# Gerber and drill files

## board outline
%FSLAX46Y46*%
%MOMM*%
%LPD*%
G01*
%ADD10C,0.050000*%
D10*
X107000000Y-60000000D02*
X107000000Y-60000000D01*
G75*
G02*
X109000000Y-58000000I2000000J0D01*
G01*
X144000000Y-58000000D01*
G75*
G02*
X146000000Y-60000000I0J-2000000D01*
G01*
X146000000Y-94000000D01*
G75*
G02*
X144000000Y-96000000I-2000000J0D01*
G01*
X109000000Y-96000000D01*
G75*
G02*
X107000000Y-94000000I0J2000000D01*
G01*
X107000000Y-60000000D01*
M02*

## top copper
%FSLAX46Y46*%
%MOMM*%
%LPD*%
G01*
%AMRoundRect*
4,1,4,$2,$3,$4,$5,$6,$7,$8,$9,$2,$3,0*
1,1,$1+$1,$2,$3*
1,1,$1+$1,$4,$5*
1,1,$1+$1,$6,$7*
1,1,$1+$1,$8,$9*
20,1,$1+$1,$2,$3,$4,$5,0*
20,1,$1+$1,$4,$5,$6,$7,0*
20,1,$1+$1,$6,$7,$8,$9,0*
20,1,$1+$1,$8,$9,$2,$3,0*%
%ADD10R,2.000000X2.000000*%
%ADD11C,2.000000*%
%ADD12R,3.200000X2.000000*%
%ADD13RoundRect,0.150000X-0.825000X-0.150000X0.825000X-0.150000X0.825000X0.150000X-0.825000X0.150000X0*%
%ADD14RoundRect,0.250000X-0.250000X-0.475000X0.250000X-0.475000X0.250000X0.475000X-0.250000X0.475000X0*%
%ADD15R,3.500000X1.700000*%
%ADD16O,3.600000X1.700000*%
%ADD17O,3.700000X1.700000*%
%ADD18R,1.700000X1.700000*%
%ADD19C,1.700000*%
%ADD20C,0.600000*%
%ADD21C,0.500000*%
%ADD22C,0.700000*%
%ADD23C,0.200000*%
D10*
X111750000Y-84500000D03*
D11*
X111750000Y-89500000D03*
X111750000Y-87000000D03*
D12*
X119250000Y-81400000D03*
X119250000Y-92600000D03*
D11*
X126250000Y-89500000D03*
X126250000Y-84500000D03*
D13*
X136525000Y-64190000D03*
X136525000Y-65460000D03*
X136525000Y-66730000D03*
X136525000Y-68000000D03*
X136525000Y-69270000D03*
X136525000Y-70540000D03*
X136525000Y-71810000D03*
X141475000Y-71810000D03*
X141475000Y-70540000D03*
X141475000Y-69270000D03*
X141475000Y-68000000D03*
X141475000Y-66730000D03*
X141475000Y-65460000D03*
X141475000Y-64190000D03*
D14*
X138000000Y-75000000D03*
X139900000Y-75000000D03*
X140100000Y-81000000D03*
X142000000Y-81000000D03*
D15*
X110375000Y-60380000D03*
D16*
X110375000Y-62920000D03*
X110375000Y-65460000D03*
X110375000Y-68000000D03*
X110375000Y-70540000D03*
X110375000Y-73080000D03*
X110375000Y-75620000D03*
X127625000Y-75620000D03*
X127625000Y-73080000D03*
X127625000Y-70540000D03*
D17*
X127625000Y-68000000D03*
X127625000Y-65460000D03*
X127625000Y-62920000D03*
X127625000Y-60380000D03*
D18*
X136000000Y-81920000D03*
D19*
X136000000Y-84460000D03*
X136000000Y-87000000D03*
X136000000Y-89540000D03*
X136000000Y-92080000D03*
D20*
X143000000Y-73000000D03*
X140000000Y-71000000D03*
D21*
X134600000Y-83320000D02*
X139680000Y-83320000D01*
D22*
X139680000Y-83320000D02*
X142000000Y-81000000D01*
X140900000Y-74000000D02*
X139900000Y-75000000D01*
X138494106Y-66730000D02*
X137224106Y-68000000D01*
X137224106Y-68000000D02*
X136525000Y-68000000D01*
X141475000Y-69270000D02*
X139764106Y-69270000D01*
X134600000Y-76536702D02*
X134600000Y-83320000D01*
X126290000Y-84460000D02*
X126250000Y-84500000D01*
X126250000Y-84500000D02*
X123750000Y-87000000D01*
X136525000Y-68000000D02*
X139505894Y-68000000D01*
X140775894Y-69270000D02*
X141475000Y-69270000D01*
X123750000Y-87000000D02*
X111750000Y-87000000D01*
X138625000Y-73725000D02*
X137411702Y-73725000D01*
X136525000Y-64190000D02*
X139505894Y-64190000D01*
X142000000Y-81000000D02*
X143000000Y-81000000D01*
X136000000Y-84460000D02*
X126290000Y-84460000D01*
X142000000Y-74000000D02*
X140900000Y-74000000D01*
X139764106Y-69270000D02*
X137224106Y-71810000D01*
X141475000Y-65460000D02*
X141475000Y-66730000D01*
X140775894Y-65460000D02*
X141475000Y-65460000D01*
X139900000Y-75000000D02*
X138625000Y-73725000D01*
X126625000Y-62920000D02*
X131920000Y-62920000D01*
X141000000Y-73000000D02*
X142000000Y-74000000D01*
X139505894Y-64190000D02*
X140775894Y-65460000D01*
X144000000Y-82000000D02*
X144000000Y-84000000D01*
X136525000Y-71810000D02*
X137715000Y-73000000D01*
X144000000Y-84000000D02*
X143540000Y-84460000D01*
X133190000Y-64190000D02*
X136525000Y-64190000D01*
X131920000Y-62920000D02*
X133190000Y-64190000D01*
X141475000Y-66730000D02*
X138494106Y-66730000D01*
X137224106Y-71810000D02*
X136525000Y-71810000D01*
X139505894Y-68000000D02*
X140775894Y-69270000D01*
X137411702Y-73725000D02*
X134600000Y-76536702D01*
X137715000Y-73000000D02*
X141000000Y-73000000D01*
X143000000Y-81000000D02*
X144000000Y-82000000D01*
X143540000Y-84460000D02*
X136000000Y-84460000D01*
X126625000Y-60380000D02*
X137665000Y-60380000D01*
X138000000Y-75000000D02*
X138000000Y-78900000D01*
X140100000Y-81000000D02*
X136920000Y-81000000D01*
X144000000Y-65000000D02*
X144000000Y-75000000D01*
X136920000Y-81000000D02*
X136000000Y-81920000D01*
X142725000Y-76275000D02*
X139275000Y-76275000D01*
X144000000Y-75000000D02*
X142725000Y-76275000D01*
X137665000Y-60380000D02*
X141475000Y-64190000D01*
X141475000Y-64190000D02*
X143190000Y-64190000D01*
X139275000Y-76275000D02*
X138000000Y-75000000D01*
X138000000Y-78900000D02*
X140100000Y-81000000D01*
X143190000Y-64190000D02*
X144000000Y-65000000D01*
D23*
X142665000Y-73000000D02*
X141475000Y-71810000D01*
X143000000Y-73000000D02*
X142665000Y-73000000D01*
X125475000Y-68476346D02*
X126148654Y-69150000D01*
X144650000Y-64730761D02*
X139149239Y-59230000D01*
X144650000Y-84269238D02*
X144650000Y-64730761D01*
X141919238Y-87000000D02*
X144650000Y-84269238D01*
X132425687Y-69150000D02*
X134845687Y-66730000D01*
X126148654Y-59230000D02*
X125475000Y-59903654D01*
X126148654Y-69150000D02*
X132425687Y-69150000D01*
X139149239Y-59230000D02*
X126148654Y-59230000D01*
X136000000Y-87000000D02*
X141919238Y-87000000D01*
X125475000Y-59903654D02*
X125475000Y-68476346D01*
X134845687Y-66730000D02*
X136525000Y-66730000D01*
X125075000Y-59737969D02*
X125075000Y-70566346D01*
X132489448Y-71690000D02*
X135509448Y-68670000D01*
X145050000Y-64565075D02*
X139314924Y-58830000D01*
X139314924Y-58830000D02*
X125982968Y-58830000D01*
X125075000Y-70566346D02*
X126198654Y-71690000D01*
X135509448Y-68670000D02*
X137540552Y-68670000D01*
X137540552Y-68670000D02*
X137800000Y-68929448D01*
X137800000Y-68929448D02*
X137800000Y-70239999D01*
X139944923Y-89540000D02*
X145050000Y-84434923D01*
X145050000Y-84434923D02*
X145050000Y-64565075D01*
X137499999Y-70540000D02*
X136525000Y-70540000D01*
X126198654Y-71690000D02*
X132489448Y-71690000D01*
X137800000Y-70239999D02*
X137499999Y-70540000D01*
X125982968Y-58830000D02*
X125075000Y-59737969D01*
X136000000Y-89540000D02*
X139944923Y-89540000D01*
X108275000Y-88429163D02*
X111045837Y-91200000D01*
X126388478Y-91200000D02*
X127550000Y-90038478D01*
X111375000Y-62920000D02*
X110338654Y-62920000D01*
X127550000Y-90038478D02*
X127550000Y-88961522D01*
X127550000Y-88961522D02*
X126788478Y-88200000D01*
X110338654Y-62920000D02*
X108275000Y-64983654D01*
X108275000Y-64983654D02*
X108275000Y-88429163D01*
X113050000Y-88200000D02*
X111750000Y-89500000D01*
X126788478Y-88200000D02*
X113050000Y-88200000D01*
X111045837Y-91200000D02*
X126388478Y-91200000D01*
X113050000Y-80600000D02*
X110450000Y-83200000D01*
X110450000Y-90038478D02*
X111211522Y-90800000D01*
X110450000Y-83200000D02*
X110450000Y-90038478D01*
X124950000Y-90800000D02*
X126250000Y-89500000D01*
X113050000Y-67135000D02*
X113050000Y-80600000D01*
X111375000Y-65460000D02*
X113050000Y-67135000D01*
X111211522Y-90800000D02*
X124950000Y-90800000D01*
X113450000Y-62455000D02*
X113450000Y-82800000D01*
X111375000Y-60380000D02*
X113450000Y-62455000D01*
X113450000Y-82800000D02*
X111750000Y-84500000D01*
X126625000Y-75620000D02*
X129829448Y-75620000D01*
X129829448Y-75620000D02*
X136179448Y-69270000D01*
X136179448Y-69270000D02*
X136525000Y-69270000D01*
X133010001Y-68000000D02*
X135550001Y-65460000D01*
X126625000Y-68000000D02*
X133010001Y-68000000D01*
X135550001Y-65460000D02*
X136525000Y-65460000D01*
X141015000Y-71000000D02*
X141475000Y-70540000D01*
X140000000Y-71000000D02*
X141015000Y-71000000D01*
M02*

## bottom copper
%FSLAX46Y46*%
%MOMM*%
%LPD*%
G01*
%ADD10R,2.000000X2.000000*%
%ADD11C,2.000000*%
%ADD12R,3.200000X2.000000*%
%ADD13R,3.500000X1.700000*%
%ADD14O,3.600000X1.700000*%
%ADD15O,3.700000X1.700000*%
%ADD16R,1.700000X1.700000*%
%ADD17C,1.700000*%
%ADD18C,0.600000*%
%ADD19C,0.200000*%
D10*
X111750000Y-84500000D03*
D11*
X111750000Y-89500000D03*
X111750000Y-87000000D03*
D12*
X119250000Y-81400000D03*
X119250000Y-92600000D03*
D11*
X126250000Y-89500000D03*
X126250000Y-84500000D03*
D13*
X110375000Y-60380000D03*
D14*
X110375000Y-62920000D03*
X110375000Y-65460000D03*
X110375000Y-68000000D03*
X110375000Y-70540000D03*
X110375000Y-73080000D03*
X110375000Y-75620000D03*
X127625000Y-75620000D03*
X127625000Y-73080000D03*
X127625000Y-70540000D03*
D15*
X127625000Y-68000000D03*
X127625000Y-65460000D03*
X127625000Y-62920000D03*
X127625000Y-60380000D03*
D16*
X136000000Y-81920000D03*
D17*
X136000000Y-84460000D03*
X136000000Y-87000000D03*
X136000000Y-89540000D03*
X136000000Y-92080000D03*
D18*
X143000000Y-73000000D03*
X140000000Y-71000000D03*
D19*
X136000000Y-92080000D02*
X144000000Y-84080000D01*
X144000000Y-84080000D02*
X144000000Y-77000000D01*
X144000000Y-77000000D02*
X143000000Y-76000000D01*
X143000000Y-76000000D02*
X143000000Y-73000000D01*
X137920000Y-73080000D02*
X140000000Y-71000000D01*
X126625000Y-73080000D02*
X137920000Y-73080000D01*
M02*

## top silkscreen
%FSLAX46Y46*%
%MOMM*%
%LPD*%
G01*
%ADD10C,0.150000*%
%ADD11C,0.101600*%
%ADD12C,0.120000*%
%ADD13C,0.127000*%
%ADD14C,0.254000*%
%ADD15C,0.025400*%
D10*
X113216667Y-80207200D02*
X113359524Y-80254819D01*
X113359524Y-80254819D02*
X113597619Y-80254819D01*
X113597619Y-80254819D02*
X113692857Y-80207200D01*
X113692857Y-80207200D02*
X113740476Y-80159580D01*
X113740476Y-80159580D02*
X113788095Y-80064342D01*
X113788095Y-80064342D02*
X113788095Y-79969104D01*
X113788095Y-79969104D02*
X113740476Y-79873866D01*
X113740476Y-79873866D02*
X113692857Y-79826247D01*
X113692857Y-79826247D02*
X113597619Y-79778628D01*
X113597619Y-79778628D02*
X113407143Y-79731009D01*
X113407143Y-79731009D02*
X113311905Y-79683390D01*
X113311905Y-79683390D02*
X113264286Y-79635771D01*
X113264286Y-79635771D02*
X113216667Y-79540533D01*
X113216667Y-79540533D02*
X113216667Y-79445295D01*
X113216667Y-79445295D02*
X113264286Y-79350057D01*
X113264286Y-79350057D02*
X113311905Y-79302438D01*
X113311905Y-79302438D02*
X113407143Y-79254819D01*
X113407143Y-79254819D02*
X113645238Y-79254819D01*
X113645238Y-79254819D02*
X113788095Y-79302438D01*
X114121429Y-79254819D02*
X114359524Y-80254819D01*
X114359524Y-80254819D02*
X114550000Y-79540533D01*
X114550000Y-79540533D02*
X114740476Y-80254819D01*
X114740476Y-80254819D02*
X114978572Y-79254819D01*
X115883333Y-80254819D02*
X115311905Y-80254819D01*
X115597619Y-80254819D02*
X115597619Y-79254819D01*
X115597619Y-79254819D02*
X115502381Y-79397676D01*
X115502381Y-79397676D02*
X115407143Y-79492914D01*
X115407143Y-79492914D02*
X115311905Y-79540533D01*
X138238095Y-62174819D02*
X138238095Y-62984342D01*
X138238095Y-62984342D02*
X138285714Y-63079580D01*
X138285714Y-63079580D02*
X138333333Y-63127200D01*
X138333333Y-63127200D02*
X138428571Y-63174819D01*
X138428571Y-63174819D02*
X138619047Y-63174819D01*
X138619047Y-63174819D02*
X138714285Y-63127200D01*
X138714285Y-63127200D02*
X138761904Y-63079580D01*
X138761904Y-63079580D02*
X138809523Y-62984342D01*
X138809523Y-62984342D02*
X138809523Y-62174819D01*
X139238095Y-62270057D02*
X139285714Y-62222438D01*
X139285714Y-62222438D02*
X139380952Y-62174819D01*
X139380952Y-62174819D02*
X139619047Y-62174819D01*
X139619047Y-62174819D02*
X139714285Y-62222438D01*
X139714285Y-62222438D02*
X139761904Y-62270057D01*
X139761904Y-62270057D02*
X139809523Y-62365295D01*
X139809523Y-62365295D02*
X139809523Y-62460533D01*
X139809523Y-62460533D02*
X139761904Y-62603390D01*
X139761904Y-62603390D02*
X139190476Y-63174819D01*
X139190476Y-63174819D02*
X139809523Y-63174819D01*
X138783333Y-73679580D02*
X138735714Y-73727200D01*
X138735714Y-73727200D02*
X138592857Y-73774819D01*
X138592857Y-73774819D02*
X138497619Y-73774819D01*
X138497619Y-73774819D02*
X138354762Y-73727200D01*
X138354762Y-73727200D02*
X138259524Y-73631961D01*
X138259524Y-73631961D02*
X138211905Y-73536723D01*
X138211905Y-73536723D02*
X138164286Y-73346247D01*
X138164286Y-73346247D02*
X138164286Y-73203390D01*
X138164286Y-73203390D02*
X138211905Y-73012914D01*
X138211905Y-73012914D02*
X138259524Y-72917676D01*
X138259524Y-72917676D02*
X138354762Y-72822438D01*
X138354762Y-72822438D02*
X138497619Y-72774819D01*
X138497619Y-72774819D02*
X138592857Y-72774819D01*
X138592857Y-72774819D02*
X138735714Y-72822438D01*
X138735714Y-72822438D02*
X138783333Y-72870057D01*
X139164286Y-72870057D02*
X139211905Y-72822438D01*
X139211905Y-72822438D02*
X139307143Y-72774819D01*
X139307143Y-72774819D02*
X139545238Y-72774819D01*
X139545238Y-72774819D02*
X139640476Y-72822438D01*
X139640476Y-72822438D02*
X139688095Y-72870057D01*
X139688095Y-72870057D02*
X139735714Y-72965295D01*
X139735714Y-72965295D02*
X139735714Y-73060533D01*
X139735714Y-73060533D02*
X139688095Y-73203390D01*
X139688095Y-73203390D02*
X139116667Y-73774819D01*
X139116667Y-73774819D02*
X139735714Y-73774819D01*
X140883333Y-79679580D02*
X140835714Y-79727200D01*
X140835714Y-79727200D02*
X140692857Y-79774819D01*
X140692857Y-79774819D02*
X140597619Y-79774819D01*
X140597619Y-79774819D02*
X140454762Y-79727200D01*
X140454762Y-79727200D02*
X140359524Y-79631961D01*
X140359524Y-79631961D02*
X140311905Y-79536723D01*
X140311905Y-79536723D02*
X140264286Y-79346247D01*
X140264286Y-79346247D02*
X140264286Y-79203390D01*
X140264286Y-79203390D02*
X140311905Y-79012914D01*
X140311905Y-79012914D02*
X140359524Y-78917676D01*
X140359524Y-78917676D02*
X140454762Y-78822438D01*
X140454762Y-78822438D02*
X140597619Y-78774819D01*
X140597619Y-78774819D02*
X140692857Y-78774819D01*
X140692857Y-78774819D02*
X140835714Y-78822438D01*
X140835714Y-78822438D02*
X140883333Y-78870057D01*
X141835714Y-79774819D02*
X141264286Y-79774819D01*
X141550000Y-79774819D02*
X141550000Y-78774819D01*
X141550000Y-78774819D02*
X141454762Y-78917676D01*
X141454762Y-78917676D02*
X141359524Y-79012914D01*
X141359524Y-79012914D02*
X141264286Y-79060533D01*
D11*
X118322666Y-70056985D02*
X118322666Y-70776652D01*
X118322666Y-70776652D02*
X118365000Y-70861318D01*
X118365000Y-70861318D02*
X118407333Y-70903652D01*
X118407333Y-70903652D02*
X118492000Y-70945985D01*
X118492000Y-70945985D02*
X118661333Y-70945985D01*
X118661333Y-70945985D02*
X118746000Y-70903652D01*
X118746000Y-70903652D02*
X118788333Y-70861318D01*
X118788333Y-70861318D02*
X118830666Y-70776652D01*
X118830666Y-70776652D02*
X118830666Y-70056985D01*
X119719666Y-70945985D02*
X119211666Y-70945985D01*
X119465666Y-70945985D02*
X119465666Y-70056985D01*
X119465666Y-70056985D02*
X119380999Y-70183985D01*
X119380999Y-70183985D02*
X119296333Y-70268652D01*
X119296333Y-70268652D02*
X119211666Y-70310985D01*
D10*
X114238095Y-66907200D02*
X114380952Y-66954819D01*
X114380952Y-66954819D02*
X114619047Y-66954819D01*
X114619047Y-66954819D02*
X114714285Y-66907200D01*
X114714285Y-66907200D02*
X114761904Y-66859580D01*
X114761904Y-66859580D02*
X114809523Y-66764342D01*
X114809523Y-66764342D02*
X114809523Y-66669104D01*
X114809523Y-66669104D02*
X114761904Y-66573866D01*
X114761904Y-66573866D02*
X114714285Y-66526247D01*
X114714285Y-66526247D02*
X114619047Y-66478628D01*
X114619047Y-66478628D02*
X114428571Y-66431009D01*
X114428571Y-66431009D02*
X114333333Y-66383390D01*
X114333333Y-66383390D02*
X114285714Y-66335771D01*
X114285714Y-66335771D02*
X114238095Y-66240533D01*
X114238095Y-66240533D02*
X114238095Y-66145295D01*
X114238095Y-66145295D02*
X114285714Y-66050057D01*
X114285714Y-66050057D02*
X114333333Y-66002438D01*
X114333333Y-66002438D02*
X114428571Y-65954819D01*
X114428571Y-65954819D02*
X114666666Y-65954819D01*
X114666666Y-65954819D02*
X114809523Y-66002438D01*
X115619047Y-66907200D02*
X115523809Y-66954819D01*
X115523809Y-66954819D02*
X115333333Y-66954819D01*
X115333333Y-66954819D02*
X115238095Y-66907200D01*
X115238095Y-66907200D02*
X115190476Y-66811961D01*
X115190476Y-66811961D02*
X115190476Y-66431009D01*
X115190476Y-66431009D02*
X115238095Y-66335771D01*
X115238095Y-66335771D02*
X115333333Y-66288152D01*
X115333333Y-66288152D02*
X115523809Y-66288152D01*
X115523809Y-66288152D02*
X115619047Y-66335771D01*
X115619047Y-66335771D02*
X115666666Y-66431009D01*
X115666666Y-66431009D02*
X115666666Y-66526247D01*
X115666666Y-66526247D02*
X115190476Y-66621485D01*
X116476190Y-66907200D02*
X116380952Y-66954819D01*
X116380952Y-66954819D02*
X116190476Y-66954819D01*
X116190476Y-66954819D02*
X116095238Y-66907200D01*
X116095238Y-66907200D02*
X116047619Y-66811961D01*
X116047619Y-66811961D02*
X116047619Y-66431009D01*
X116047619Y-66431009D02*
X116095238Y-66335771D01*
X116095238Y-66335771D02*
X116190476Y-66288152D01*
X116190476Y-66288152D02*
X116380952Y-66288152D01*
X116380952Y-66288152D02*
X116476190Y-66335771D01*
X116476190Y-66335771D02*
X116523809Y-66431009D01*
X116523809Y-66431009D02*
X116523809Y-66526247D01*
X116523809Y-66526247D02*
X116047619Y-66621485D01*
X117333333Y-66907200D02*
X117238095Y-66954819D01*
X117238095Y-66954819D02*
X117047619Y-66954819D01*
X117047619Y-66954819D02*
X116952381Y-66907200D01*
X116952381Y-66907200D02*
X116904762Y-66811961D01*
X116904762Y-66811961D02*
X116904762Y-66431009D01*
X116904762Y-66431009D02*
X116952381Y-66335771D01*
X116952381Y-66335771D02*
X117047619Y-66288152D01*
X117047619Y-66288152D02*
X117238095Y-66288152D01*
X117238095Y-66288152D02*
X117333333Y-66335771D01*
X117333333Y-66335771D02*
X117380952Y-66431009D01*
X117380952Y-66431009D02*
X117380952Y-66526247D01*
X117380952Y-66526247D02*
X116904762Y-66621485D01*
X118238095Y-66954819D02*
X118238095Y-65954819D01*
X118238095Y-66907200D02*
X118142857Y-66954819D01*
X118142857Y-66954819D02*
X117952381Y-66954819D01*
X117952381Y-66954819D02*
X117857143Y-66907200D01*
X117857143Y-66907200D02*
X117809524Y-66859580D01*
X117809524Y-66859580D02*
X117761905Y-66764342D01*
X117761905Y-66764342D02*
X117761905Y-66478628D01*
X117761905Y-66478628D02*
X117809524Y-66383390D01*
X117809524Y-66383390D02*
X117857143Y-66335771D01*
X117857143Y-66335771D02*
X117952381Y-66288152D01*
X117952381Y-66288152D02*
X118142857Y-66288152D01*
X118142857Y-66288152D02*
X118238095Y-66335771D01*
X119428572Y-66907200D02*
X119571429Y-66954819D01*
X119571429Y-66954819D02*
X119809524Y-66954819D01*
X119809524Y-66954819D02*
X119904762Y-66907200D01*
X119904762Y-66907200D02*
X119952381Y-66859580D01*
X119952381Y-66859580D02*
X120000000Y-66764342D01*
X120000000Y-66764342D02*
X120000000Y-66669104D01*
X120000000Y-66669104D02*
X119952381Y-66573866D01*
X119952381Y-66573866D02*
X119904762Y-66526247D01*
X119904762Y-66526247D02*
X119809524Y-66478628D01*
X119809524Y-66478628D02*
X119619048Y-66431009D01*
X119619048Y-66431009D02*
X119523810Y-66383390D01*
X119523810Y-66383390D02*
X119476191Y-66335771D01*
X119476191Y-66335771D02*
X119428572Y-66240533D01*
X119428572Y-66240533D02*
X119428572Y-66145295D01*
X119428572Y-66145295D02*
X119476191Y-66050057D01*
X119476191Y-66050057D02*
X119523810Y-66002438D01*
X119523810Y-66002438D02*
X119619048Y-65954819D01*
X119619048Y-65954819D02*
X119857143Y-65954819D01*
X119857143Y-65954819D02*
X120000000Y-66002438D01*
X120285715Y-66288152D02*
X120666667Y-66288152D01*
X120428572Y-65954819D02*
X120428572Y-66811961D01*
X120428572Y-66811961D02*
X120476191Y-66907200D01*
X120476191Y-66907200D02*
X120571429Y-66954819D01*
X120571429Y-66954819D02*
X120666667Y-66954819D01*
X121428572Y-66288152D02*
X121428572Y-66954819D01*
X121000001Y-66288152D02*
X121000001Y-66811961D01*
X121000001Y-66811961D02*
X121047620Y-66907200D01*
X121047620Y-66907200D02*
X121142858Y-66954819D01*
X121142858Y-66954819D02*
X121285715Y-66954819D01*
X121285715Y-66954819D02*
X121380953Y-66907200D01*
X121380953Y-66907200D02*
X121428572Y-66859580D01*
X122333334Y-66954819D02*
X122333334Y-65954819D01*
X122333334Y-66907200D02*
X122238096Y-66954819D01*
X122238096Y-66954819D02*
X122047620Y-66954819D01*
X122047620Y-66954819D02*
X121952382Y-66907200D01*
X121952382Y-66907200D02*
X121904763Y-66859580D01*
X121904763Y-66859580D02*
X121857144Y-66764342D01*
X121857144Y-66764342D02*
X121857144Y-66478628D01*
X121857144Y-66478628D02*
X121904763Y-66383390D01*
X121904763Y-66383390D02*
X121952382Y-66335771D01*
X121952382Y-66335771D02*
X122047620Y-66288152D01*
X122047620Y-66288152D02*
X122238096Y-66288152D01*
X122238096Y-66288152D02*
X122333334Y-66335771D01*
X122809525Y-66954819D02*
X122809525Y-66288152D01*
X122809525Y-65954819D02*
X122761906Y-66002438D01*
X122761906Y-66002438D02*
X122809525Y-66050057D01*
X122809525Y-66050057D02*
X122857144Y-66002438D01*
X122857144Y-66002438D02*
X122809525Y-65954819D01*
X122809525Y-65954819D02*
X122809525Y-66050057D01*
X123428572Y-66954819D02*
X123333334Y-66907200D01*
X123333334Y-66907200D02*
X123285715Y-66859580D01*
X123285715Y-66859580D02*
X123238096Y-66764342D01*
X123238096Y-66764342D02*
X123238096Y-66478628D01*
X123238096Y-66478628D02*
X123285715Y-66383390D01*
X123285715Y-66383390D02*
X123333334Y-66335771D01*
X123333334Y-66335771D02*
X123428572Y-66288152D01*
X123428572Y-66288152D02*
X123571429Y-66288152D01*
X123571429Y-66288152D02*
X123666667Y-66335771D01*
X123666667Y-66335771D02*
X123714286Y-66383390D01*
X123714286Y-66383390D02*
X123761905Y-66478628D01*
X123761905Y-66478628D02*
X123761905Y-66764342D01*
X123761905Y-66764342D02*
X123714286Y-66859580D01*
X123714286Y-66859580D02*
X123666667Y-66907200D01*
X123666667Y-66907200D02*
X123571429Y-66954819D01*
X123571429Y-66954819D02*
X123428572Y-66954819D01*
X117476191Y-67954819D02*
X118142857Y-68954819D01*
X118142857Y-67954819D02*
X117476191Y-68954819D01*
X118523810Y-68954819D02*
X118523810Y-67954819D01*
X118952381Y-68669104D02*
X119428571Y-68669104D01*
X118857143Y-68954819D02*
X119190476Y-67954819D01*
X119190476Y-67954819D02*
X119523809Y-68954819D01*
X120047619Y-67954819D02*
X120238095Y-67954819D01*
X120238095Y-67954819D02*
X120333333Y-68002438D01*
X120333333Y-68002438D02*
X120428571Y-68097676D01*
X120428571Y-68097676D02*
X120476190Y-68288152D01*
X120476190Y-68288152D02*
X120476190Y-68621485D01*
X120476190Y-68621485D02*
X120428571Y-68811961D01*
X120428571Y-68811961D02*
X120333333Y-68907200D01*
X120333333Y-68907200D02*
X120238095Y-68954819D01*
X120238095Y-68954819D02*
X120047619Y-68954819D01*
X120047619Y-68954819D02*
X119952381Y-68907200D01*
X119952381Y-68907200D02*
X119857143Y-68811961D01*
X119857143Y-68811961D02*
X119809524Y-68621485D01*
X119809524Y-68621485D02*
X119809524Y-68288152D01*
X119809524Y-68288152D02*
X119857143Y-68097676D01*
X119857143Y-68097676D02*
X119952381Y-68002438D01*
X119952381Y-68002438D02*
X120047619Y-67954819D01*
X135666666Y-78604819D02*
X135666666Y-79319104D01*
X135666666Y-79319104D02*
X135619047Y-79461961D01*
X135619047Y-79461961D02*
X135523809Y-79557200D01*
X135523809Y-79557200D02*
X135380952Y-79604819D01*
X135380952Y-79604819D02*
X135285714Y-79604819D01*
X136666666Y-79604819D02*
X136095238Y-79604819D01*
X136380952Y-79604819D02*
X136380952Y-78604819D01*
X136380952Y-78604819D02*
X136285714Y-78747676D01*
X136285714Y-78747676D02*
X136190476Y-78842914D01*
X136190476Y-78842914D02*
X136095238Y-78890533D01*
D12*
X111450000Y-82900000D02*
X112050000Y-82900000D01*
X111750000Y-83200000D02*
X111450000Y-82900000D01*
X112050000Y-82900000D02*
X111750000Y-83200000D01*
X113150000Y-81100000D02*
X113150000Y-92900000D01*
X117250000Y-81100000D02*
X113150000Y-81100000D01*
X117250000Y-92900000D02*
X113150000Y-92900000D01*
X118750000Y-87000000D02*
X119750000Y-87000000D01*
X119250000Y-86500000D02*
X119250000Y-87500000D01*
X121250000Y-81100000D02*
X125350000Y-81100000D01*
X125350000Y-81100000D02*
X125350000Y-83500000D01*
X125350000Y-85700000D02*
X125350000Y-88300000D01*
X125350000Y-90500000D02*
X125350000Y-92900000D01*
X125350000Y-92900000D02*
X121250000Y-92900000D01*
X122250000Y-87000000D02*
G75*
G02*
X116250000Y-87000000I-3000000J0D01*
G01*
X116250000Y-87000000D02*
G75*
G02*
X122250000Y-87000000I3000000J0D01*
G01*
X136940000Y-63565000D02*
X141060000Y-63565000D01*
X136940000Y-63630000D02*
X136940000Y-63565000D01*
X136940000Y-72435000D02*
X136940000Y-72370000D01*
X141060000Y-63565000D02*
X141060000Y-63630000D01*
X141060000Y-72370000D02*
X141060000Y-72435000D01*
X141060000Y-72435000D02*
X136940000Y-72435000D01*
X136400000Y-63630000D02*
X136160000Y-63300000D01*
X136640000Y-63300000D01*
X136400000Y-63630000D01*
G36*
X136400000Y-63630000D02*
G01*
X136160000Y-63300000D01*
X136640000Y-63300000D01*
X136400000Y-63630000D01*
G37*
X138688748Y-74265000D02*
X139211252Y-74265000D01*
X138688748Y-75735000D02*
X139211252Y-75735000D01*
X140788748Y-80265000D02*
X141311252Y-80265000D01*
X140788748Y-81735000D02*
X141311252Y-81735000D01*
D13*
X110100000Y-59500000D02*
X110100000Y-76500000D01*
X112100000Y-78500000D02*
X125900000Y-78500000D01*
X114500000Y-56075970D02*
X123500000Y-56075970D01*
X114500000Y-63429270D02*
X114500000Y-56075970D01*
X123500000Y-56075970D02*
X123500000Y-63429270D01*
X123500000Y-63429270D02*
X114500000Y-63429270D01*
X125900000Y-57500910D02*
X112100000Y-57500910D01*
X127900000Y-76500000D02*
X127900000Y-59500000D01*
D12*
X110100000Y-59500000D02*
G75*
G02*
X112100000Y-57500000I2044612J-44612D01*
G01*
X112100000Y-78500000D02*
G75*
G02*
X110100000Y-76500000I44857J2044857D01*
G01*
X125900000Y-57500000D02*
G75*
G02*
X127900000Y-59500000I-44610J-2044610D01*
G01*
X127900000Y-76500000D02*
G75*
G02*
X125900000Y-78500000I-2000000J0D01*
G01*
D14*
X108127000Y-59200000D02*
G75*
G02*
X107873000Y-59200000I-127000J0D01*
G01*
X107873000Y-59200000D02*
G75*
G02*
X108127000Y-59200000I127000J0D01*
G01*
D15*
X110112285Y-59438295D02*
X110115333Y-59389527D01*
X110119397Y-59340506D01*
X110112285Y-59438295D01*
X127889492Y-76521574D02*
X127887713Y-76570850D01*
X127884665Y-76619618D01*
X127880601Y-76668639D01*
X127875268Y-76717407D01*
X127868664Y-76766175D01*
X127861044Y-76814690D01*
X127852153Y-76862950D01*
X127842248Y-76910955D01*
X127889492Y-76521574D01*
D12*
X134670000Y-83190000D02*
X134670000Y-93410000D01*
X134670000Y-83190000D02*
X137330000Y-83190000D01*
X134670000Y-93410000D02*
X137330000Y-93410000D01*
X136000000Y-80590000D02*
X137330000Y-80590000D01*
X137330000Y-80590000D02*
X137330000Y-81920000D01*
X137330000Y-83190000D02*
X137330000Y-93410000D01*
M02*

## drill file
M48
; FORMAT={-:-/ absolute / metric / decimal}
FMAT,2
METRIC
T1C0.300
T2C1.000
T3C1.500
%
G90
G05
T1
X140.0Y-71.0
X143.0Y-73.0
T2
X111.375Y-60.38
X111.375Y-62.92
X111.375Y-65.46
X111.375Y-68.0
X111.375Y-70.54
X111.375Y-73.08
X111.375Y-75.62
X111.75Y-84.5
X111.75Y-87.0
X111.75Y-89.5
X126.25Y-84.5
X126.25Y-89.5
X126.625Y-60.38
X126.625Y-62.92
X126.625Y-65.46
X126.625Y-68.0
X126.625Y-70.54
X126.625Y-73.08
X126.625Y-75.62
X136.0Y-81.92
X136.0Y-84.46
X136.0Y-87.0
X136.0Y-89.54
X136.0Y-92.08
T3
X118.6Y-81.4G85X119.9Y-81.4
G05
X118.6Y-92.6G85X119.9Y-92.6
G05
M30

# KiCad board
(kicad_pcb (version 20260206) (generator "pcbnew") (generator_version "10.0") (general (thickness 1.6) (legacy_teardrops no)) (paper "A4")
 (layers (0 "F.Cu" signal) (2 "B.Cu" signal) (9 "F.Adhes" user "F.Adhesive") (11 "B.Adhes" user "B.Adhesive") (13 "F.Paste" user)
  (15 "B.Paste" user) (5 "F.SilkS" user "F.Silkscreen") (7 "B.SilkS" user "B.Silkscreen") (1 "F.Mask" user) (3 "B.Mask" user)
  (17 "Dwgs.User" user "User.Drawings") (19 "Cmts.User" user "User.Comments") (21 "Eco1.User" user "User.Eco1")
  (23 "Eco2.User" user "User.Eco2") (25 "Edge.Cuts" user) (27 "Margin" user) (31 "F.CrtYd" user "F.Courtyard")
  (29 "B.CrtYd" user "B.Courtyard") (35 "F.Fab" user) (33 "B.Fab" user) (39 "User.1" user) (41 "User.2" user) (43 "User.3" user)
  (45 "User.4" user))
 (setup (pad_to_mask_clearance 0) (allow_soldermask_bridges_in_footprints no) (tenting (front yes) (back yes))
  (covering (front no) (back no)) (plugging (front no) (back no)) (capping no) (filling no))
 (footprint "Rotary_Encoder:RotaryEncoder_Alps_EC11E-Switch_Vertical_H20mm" (layer "F.Cu") (at 111.75 84.5)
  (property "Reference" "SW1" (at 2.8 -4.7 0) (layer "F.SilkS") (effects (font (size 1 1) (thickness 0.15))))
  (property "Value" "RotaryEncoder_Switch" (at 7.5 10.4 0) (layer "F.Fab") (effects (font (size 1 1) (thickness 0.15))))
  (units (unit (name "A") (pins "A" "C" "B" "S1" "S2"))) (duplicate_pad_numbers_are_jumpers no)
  (fp_line (start -0.3 -1.6) (end 0.3 -1.6) (stroke (width 0.12) (type solid)) (layer "F.SilkS"))
  (fp_line (start 0 -1.3) (end -0.3 -1.6) (stroke (width 0.12) (type solid)) (layer "F.SilkS"))
  (fp_line (start 0.3 -1.6) (end 0 -1.3) (stroke (width 0.12) (type solid)) (layer "F.SilkS"))
  (fp_line (start 1.4 -3.4) (end 1.4 8.4) (stroke (width 0.12) (type solid)) (layer "F.SilkS"))
  (fp_line (start 5.5 -3.4) (end 1.4 -3.4) (stroke (width 0.12) (type solid)) (layer "F.SilkS"))
  (fp_line (start 5.5 8.4) (end 1.4 8.4) (stroke (width 0.12) (type solid)) (layer "F.SilkS"))
  (fp_line (start 7 2.5) (end 8 2.5) (stroke (width 0.12) (type solid)) (layer "F.SilkS"))
  (fp_line (start 7.5 2) (end 7.5 3) (stroke (width 0.12) (type solid)) (layer "F.SilkS"))
  (fp_line (start 9.5 -3.4) (end 13.6 -3.4) (stroke (width 0.12) (type solid)) (layer "F.SilkS"))
  (fp_line (start 13.6 -3.4) (end 13.6 -1) (stroke (width 0.12) (type solid)) (layer "F.SilkS"))
  (fp_line (start 13.6 1.2) (end 13.6 3.8) (stroke (width 0.12) (type solid)) (layer "F.SilkS"))
  (fp_line (start 13.6 6) (end 13.6 8.4) (stroke (width 0.12) (type solid)) (layer "F.SilkS"))
  (fp_line (start 13.6 8.4) (end 9.5 8.4) (stroke (width 0.12) (type solid)) (layer "F.SilkS"))
  (fp_circle (center 7.5 2.5) (end 10.5 2.5) (stroke (width 0.12) (type solid)) (fill no) (layer "F.SilkS"))
  (pad "A" thru_hole rect (at 0 0) (size 2 2) (drill 1) (layers "*.Cu" "*.Mask") (remove_unused_layers no) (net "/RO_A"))
  (pad "B" thru_hole circle (at 0 5) (size 2 2) (drill 1) (layers "*.Cu" "*.Mask") (remove_unused_layers no) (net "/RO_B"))
  (pad "C" thru_hole circle (at 0 2.5) (size 2 2) (drill 1) (layers "*.Cu" "*.Mask") (remove_unused_layers no) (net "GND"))
  (pad "MP" thru_hole rect (at 7.5 -3.1) (size 3.2 2) (drill oval 2.8 1.5) (layers "*.Cu" "*.Mask") (remove_unused_layers no))
  (pad "MP" thru_hole rect (at 7.5 8.1) (size 3.2 2) (drill oval 2.8 1.5) (layers "*.Cu" "*.Mask") (remove_unused_layers no))
  (pad "S1" thru_hole circle (at 14.5 5) (size 2 2) (drill 1) (layers "*.Cu" "*.Mask") (remove_unused_layers no) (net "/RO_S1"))
  (pad "S2" thru_hole circle (at 14.5 0) (size 2 2) (drill 1) (layers "*.Cu" "*.Mask") (remove_unused_layers no) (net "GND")))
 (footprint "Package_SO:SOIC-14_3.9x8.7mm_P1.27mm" (layer "F.Cu") (at 139 68)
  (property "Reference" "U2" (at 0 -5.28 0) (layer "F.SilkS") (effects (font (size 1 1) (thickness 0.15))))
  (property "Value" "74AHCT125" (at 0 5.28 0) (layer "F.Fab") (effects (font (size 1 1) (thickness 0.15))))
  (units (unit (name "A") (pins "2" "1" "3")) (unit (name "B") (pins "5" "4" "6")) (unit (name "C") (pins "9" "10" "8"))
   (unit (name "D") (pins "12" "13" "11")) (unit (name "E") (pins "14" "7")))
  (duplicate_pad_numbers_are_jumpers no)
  (fp_line (start -2.06 -4.435) (end 2.06 -4.435) (stroke (width 0.12) (type solid)) (layer "F.SilkS"))
  (fp_line (start -2.06 -4.37) (end -2.06 -4.435) (stroke (width 0.12) (type solid)) (layer "F.SilkS"))
  (fp_line (start -2.06 4.435) (end -2.06 4.37) (stroke (width 0.12) (type solid)) (layer "F.SilkS"))
  (fp_line (start 2.06 -4.435) (end 2.06 -4.37) (stroke (width 0.12) (type solid)) (layer "F.SilkS"))
  (fp_line (start 2.06 4.37) (end 2.06 4.435) (stroke (width 0.12) (type solid)) (layer "F.SilkS"))
  (fp_line (start 2.06 4.435) (end -2.06 4.435) (stroke (width 0.12) (type solid)) (layer "F.SilkS"))
  (fp_poly (pts (xy -2.6 -4.37) (xy -2.84 -4.7) (xy -2.36 -4.7)) (stroke (width 0.12) (type solid)) (fill yes) (layer "F.SilkS"))
  (pad "1" smd roundrect (at -2.475 -3.81) (size 1.95 0.6) (layers "F.Cu" "F.Mask" "F.Paste") (roundrect_rratio 0.25) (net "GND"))
  (pad "2" smd roundrect (at -2.475 -2.54) (size 1.95 0.6) (layers "F.Cu" "F.Mask" "F.Paste") (roundrect_rratio 0.25) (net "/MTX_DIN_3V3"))
  (pad "3" smd roundrect (at -2.475 -1.27) (size 1.95 0.6) (layers "F.Cu" "F.Mask" "F.Paste") (roundrect_rratio 0.25) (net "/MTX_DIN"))
  (pad "4" smd roundrect (at -2.475 0) (size 1.95 0.6) (layers "F.Cu" "F.Mask" "F.Paste") (roundrect_rratio 0.25) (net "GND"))
  (pad "5" smd roundrect (at -2.475 1.27) (size 1.95 0.6) (layers "F.Cu" "F.Mask" "F.Paste") (roundrect_rratio 0.25) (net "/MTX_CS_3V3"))
  (pad "6" smd roundrect (at -2.475 2.54) (size 1.95 0.6) (layers "F.Cu" "F.Mask" "F.Paste") (roundrect_rratio 0.25) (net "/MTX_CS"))
  (pad "7" smd roundrect (at -2.475 3.81) (size 1.95 0.6) (layers "F.Cu" "F.Mask" "F.Paste") (roundrect_rratio 0.25) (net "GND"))
  (pad "8" smd roundrect (at 2.475 3.81) (size 1.95 0.6) (layers "F.Cu" "F.Mask" "F.Paste") (roundrect_rratio 0.25) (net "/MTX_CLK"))
  (pad "9" smd roundrect (at 2.475 2.54) (size 1.95 0.6) (layers "F.Cu" "F.Mask" "F.Paste") (roundrect_rratio 0.25) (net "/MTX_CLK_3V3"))
  (pad "10" smd roundrect (at 2.475 1.27) (size 1.95 0.6) (layers "F.Cu" "F.Mask" "F.Paste") (roundrect_rratio 0.25) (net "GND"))
  (pad "11" smd roundrect (at 2.475 0) (size 1.95 0.6) (layers "F.Cu" "F.Mask" "F.Paste") (roundrect_rratio 0.25)
   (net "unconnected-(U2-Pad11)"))
  (pad "12" smd roundrect (at 2.475 -1.27) (size 1.95 0.6) (layers "F.Cu" "F.Mask" "F.Paste") (roundrect_rratio 0.25) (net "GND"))
  (pad "13" smd roundrect (at 2.475 -2.54) (size 1.95 0.6) (layers "F.Cu" "F.Mask" "F.Paste") (roundrect_rratio 0.25) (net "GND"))
  (pad "14" smd roundrect (at 2.475 -3.81) (size 1.95 0.6) (layers "F.Cu" "F.Mask" "F.Paste") (roundrect_rratio 0.25) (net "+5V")))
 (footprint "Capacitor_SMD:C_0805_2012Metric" (layer "F.Cu") (at 138.95 75)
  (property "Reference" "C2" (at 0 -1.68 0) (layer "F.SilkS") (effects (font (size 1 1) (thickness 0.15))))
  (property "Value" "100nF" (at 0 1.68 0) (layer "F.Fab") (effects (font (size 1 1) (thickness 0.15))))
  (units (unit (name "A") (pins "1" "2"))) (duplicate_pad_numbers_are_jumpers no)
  (fp_line (start -0.261252 -0.735) (end 0.261252 -0.735) (stroke (width 0.12) (type solid)) (layer "F.SilkS"))
  (fp_line (start -0.261252 0.735) (end 0.261252 0.735) (stroke (width 0.12) (type solid)) (layer "F.SilkS"))
  (pad "1" smd roundrect (at -0.95 0) (size 1 1.45) (layers "F.Cu" "F.Mask" "F.Paste") (roundrect_rratio 0.25) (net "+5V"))
  (pad "2" smd roundrect (at 0.95 0) (size 1 1.45) (layers "F.Cu" "F.Mask" "F.Paste") (roundrect_rratio 0.25) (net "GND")))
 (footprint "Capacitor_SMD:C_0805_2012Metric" (layer "F.Cu") (at 141.05 81)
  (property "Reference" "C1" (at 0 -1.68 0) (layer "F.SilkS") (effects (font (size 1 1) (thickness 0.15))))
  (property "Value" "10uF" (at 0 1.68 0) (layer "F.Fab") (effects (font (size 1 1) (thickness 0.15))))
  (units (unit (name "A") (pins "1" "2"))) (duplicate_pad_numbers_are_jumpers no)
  (fp_line (start -0.261252 -0.735) (end 0.261252 -0.735) (stroke (width 0.12) (type solid)) (layer "F.SilkS"))
  (fp_line (start -0.261252 0.735) (end 0.261252 0.735) (stroke (width 0.12) (type solid)) (layer "F.SilkS"))
  (pad "1" smd roundrect (at -0.95 0) (size 1 1.45) (layers "F.Cu" "F.Mask" "F.Paste") (roundrect_rratio 0.25) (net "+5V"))
  (pad "2" smd roundrect (at 0.95 0) (size 1 1.45) (layers "F.Cu" "F.Mask" "F.Paste") (roundrect_rratio 0.25) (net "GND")))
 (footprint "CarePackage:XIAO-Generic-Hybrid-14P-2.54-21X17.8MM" (layer "F.Cu") (at 119 68)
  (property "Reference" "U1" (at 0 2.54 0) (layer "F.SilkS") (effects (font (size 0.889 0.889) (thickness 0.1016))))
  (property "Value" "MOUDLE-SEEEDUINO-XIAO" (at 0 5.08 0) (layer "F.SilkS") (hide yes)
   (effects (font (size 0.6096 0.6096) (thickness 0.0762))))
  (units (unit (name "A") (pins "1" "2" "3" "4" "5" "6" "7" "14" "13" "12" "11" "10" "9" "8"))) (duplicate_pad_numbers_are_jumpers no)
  (fp_line (start -8.9 -8.5) (end -8.9 8.5) (stroke (width 0.127) (type solid)) (layer "F.SilkS"))
  (fp_line (start -6.9 10.5) (end 6.9 10.5) (stroke (width 0.127) (type solid)) (layer "F.SilkS"))
  (fp_line (start -4.5 -11.92403) (end 4.5 -11.92403) (stroke (width 0.127) (type solid)) (layer "F.SilkS"))
  (fp_line (start -4.5 -4.57073) (end -4.5 -11.92403) (stroke (width 0.127) (type solid)) (layer "F.SilkS"))
  (fp_line (start 4.5 -11.92403) (end 4.5 -4.57073) (stroke (width 0.127) (type solid)) (layer "F.SilkS"))
  (fp_line (start 4.5 -4.57073) (end -4.5 -4.57073) (stroke (width 0.127) (type solid)) (layer "F.SilkS"))
  (fp_line (start 6.9 -10.49909) (end -6.9 -10.49909) (stroke (width 0.127) (type solid)) (layer "F.SilkS"))
  (fp_line (start 8.9 8.5) (end 8.9 -8.5) (stroke (width 0.127) (type solid)) (layer "F.SilkS"))
  (fp_arc (start -8.9 -8.5) (mid -8.301491 -9.901491) (end -6.9 -10.5) (stroke (width 0.12) (type solid)) (layer "F.SilkS"))
  (fp_arc (start -6.9 10.5) (mid -8.301423 9.901423) (end -8.9 8.5) (stroke (width 0.12) (type solid)) (layer "F.SilkS"))
  (fp_arc (start 6.9 -10.5) (mid 8.301491 -9.901491) (end 8.9 -8.5) (stroke (width 0.12) (type solid)) (layer "F.SilkS"))
  (fp_arc (start 8.9 8.5) (mid 8.314214 9.914214) (end 6.9 10.5) (stroke (width 0.12) (type solid)) (layer "F.SilkS"))
  (fp_circle (center -11 -8.8) (end -11 -9.054) (stroke (width 0) (type solid)) (fill yes) (layer "F.SilkS"))
  (fp_poly
   (pts (xy -8.887715 -8.561705) (xy -8.884667 -8.610473) (xy -8.880603 -8.659494)) (stroke (width 0.0254) (type solid)) (fill no)
   (layer "F.SilkS"))
  (fp_poly
   (pts (xy 8.889492 8.521574) (xy 8.887713 8.57085) (xy 8.884665 8.619618) (xy 8.880601 8.668639) (xy 8.875268 8.717407)
    (xy 8.868664 8.766175) (xy 8.861044 8.81469) (xy 8.852153 8.86295) (xy 8.842248 8.910955))
   (stroke (width 0.0254) (type solid)) (fill no) (layer "F.SilkS"))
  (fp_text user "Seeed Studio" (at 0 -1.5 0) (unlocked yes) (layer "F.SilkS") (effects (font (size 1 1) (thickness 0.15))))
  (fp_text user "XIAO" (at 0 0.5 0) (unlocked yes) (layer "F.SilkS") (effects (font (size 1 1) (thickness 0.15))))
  (pad "1" thru_hole rect (at -7.625 -7.62) (size 3.5 1.7) (drill 1 (offset -1 0)) (layers "*.Cu" "*.Mask") (remove_unused_layers no)
   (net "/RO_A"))
  (pad "2" thru_hole oval (at -7.625 -5.08) (size 3.6 1.7) (drill 1 (offset -1 0)) (layers "*.Cu" "*.Mask") (remove_unused_layers no)
   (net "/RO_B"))
  (pad "3" thru_hole oval (at -7.625 -2.54) (size 3.6 1.7) (drill 1 (offset -1 0)) (layers "*.Cu" "*.Mask") (remove_unused_layers no)
   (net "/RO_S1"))
  (pad "4" thru_hole oval (at -7.625 0) (size 3.6 1.7) (drill 1 (offset -1 0)) (layers "*.Cu" "*.Mask") (remove_unused_layers no)
   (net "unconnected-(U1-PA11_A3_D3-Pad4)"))
  (pad "5" thru_hole oval (at -7.625 2.54) (size 3.6 1.7) (drill 1 (offset -1 0)) (layers "*.Cu" "*.Mask") (remove_unused_layers no)
   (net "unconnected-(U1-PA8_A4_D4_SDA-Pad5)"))
  (pad "6" thru_hole oval (at -7.625 5.08 180) (size 3.6 1.7) (drill 1 (offset 1 0)) (layers "*.Cu" "*.Mask") (remove_unused_layers no)
   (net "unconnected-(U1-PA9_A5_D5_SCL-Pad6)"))
  (pad "7" thru_hole oval (at -7.625 7.62) (size 3.6 1.7) (drill 1 (offset -1 0)) (layers "*.Cu" "*.Mask") (remove_unused_layers no)
   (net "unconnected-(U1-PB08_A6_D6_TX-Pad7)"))
  (pad "8" thru_hole oval (at 7.625 7.62) (size 3.6 1.7) (drill 1 (offset 1 0)) (layers "*.Cu" "*.Mask") (remove_unused_layers no)
   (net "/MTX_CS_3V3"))
  (pad "9" thru_hole oval (at 7.625 5.08) (size 3.6 1.7) (drill 1 (offset 1 0)) (layers "*.Cu" "*.Mask") (remove_unused_layers no)
   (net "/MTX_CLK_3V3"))
  (pad "10" thru_hole oval (at 7.625 2.54) (size 3.6 1.7) (drill 1 (offset 1 0)) (layers "*.Cu" "*.Mask") (remove_unused_layers no)
   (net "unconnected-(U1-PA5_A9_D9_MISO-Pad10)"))
  (pad "11" thru_hole oval (at 7.625 0) (size 3.7 1.7) (drill 1 (offset 1 0)) (layers "*.Cu" "*.Mask") (remove_unused_layers no)
   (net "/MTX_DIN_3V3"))
  (pad "12" thru_hole oval (at 7.625 -2.54) (size 3.7 1.7) (drill 1 (offset 1 0)) (layers "*.Cu" "*.Mask") (remove_unused_layers no)
   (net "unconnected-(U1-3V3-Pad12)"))
  (pad "13" thru_hole oval (at 7.625 -5.08) (size 3.7 1.7) (drill 1 (offset 1 0)) (layers "*.Cu" "*.Mask") (remove_unused_layers no)
   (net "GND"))
  (pad "14" thru_hole oval (at 7.625 -7.62) (size 3.7 1.7) (drill 1 (offset 1 0)) (layers "*.Cu" "*.Mask") (remove_unused_layers no)
   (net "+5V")))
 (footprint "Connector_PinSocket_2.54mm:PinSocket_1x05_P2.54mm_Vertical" (layer "F.Cu") (at 136 81.92)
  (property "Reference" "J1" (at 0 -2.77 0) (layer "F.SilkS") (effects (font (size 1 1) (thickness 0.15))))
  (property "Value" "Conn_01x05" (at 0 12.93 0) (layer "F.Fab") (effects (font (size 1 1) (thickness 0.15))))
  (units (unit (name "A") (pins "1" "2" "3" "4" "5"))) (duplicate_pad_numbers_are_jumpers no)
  (fp_line (start -1.33 1.27) (end -1.33 11.49) (stroke (width 0.12) (type solid)) (layer "F.SilkS"))
  (fp_line (start -1.33 1.27) (end 1.33 1.27) (stroke (width 0.12) (type solid)) (layer "F.SilkS"))
  (fp_line (start -1.33 11.49) (end 1.33 11.49) (stroke (width 0.12) (type solid)) (layer "F.SilkS"))
  (fp_line (start 0 -1.33) (end 1.33 -1.33) (stroke (width 0.12) (type solid)) (layer "F.SilkS"))
  (fp_line (start 1.33 -1.33) (end 1.33 0) (stroke (width 0.12) (type solid)) (layer "F.SilkS"))
  (fp_line (start 1.33 1.27) (end 1.33 11.49) (stroke (width 0.12) (type solid)) (layer "F.SilkS"))
  (pad "1" thru_hole rect (at 0 0) (size 1.7 1.7) (drill 1) (layers "*.Cu" "*.Mask") (remove_unused_layers no) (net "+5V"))
  (pad "2" thru_hole circle (at 0 2.54) (size 1.7 1.7) (drill 1) (layers "*.Cu" "*.Mask") (remove_unused_layers no) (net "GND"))
  (pad "3" thru_hole circle (at 0 5.08) (size 1.7 1.7) (drill 1) (layers "*.Cu" "*.Mask") (remove_unused_layers no) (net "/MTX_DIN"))
  (pad "4" thru_hole circle (at 0 7.62) (size 1.7 1.7) (drill 1) (layers "*.Cu" "*.Mask") (remove_unused_layers no) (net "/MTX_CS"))
  (pad "5" thru_hole circle (at 0 10.16) (size 1.7 1.7) (drill 1) (layers "*.Cu" "*.Mask") (remove_unused_layers no) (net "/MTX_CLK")))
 (gr_rect (start 107 58) (end 146 96) (radius 2) (stroke (width 0.05) (type default)) (fill no) (layer "Edge.Cuts"))
 (segment (start 134.6 83.32) (end 139.68 83.32) (width 0.5) (layer "F.Cu") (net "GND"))
 (segment (start 139.68 83.32) (end 142 81) (width 0.7) (layer "F.Cu") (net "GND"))
 (segment (start 140.9 74) (end 139.9 75) (width 0.7) (layer "F.Cu") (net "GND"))
 (segment (start 138.494106 66.73) (end 137.224106 68) (width 0.7) (layer "F.Cu") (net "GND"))
 (segment (start 137.224106 68) (end 136.525 68) (width 0.7) (layer "F.Cu") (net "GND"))
 (segment (start 141.475 69.27) (end 139.764106 69.27) (width 0.7) (layer "F.Cu") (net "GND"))
 (segment (start 134.6 76.536702) (end 134.6 83.32) (width 0.7) (layer "F.Cu") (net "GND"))
 (segment (start 126.29 84.46) (end 126.25 84.5) (width 0.7) (layer "F.Cu") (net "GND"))
 (segment (start 126.25 84.5) (end 123.75 87) (width 0.7) (layer "F.Cu") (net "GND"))
 (segment (start 136.525 68) (end 139.505894 68) (width 0.7) (layer "F.Cu") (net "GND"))
 (segment (start 140.775894 69.27) (end 141.475 69.27) (width 0.7) (layer "F.Cu") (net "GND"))
 (segment (start 123.75 87) (end 111.75 87) (width 0.7) (layer "F.Cu") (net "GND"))
 (segment (start 138.625 73.725) (end 137.411702 73.725) (width 0.7) (layer "F.Cu") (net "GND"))
 (segment (start 136.525 64.19) (end 139.505894 64.19) (width 0.7) (layer "F.Cu") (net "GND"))
 (segment (start 142 81) (end 143 81) (width 0.7) (layer "F.Cu") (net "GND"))
 (segment (start 136 84.46) (end 126.29 84.46) (width 0.7) (layer "F.Cu") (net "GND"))
 (segment (start 142 74) (end 140.9 74) (width 0.7) (layer "F.Cu") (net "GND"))
 (segment (start 139.764106 69.27) (end 137.224106 71.81) (width 0.7) (layer "F.Cu") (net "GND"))
 (segment (start 141.475 65.46) (end 141.475 66.73) (width 0.7) (layer "F.Cu") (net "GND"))
 (segment (start 140.775894 65.46) (end 141.475 65.46) (width 0.7) (layer "F.Cu") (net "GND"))
 (segment (start 139.9 75) (end 138.625 73.725) (width 0.7) (layer "F.Cu") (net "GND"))
 (segment (start 126.625 62.92) (end 131.92 62.92) (width 0.7) (layer "F.Cu") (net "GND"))
 (segment (start 141 73) (end 142 74) (width 0.7) (layer "F.Cu") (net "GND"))
 (segment (start 139.505894 64.19) (end 140.775894 65.46) (width 0.7) (layer "F.Cu") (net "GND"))
 (segment (start 144 82) (end 144 84) (width 0.7) (layer "F.Cu") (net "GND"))
 (segment (start 136.525 71.81) (end 137.715 73) (width 0.7) (layer "F.Cu") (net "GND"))
 (segment (start 144 84) (end 143.54 84.46) (width 0.7) (layer "F.Cu") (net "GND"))
 (segment (start 133.19 64.19) (end 136.525 64.19) (width 0.7) (layer "F.Cu") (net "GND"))
 (segment (start 131.92 62.92) (end 133.19 64.19) (width 0.7) (layer "F.Cu") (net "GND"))
 (segment (start 141.475 66.73) (end 138.494106 66.73) (width 0.7) (layer "F.Cu") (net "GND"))
 (segment (start 137.224106 71.81) (end 136.525 71.81) (width 0.7) (layer "F.Cu") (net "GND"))
 (segment (start 139.505894 68) (end 140.775894 69.27) (width 0.7) (layer "F.Cu") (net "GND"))
 (segment (start 137.411702 73.725) (end 134.6 76.536702) (width 0.7) (layer "F.Cu") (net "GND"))
 (segment (start 137.715 73) (end 141 73) (width 0.7) (layer "F.Cu") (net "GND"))
 (segment (start 143 81) (end 144 82) (width 0.7) (layer "F.Cu") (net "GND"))
 (segment (start 143.54 84.46) (end 136 84.46) (width 0.7) (layer "F.Cu") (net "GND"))
 (segment (start 126.625 60.38) (end 137.665 60.38) (width 0.7) (layer "F.Cu") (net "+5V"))
 (segment (start 138 75) (end 138 78.9) (width 0.7) (layer "F.Cu") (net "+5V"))
 (segment (start 140.1 81) (end 136.92 81) (width 0.7) (layer "F.Cu") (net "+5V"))
 (segment (start 144 65) (end 144 75) (width 0.7) (layer "F.Cu") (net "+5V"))
 (segment (start 136.92 81) (end 136 81.92) (width 0.7) (layer "F.Cu") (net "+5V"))
 (segment (start 142.725 76.275) (end 139.275 76.275) (width 0.7) (layer "F.Cu") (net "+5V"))
 (segment (start 144 75) (end 142.725 76.275) (width 0.7) (layer "F.Cu") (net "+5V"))
 (segment (start 137.665 60.38) (end 141.475 64.19) (width 0.7) (layer "F.Cu") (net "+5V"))
 (segment (start 141.475 64.19) (end 143.19 64.19) (width 0.7) (layer "F.Cu") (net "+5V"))
 (segment (start 139.275 76.275) (end 138 75) (width 0.7) (layer "F.Cu") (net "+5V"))
 (segment (start 138 78.9) (end 140.1 81) (width 0.7) (layer "F.Cu") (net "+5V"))
 (segment (start 143.19 64.19) (end 144 65) (width 0.7) (layer "F.Cu") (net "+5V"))
 (segment (start 142.665 73) (end 141.475 71.81) (width 0.2) (layer "F.Cu") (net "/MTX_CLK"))
 (segment (start 143 73) (end 142.665 73) (width 0.2) (layer "F.Cu") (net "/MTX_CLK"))
 (via (at 143 73) (size 0.6) (drill 0.3) (layers "F.Cu" "B.Cu") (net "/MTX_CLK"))
 (segment (start 136 92.08) (end 144 84.08) (width 0.2) (layer "B.Cu") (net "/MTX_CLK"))
 (segment (start 144 84.08) (end 144 77) (width 0.2) (layer "B.Cu") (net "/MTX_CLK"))
 (segment (start 144 77) (end 143 76) (width 0.2) (layer "B.Cu") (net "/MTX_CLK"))
 (segment (start 143 76) (end 143 73) (width 0.2) (layer "B.Cu") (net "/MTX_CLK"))
 (segment (start 125.475 68.476346) (end 126.148654 69.15) (width 0.2) (layer "F.Cu") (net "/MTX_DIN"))
 (segment (start 144.65 64.730761) (end 139.149239 59.23) (width 0.2) (layer "F.Cu") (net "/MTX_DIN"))
 (segment (start 144.65 84.269238) (end 144.65 64.730761) (width 0.2) (layer "F.Cu") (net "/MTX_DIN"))
 (segment (start 141.919238 87) (end 144.65 84.269238) (width 0.2) (layer "F.Cu") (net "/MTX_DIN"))
 (segment (start 132.425687 69.15) (end 134.845687 66.73) (width 0.2) (layer "F.Cu") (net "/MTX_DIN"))
 (segment (start 126.148654 59.23) (end 125.475 59.903654) (width 0.2) (layer "F.Cu") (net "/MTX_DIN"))
 (segment (start 126.148654 69.15) (end 132.425687 69.15) (width 0.2) (layer "F.Cu") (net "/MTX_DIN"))
 (segment (start 139.149239 59.23) (end 126.148654 59.23) (width 0.2) (layer "F.Cu") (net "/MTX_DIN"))
 (segment (start 136 87) (end 141.919238 87) (width 0.2) (layer "F.Cu") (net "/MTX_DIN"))
 (segment (start 125.475 59.903654) (end 125.475 68.476346) (width 0.2) (layer "F.Cu") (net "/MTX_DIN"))
 (segment (start 134.845687 66.73) (end 136.525 66.73) (width 0.2) (layer "F.Cu") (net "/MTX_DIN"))
 (segment (start 125.075 59.737969) (end 125.075 70.566346) (width 0.2) (layer "F.Cu") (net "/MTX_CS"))
 (segment (start 132.489448 71.69) (end 135.509448 68.67) (width 0.2) (layer "F.Cu") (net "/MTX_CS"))
 (segment (start 145.05 64.565075) (end 139.314924 58.83) (width 0.2) (layer "F.Cu") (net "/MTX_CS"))
 (segment (start 139.314924 58.83) (end 125.982968 58.83) (width 0.2) (layer "F.Cu") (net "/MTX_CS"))
 (segment (start 125.075 70.566346) (end 126.198654 71.69) (width 0.2) (layer "F.Cu") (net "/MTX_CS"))
 (segment (start 135.509448 68.67) (end 137.540552 68.67) (width 0.2) (layer "F.Cu") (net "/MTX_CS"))
 (segment (start 137.540552 68.67) (end 137.8 68.929448) (width 0.2) (layer "F.Cu") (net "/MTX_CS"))
 (segment (start 137.8 68.929448) (end 137.8 70.239999) (width 0.2) (layer "F.Cu") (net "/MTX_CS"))
 (segment (start 139.944923 89.54) (end 145.05 84.434923) (width 0.2) (layer "F.Cu") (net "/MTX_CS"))
 (segment (start 145.05 84.434923) (end 145.05 64.565075) (width 0.2) (layer "F.Cu") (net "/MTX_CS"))
 (segment (start 137.499999 70.54) (end 136.525 70.54) (width 0.2) (layer "F.Cu") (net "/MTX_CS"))
 (segment (start 126.198654 71.69) (end 132.489448 71.69) (width 0.2) (layer "F.Cu") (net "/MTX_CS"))
 (segment (start 137.8 70.239999) (end 137.499999 70.54) (width 0.2) (layer "F.Cu") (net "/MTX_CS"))
 (segment (start 125.982968 58.83) (end 125.075 59.737969) (width 0.2) (layer "F.Cu") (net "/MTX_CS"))
 (segment (start 136 89.54) (end 139.944923 89.54) (width 0.2) (layer "F.Cu") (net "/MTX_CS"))
 (segment (start 108.275 88.429163) (end 111.045837 91.2) (width 0.2) (layer "F.Cu") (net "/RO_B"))
 (segment (start 126.388478 91.2) (end 127.55 90.038478) (width 0.2) (layer "F.Cu") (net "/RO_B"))
 (segment (start 111.375 62.92) (end 110.338654 62.92) (width 0.2) (layer "F.Cu") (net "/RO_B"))
 (segment (start 127.55 90.038478) (end 127.55 88.961522) (width 0.2) (layer "F.Cu") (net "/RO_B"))
 (segment (start 127.55 88.961522) (end 126.788478 88.2) (width 0.2) (layer "F.Cu") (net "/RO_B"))
 (segment (start 110.338654 62.92) (end 108.275 64.983654) (width 0.2) (layer "F.Cu") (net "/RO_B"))
 (segment (start 108.275 64.983654) (end 108.275 88.429163) (width 0.2) (layer "F.Cu") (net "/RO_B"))
 (segment (start 113.05 88.2) (end 111.75 89.5) (width 0.2) (layer "F.Cu") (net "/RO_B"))
 (segment (start 126.788478 88.2) (end 113.05 88.2) (width 0.2) (layer "F.Cu") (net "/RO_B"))
 (segment (start 111.045837 91.2) (end 126.388478 91.2) (width 0.2) (layer "F.Cu") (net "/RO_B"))
 (segment (start 113.05 80.6) (end 110.45 83.2) (width 0.2) (layer "F.Cu") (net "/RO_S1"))
 (segment (start 110.45 90.038478) (end 111.211522 90.8) (width 0.2) (layer "F.Cu") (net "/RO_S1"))
 (segment (start 110.45 83.2) (end 110.45 90.038478) (width 0.2) (layer "F.Cu") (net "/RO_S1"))
 (segment (start 124.95 90.8) (end 126.25 89.5) (width 0.2) (layer "F.Cu") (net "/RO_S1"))
 (segment (start 113.05 67.135) (end 113.05 80.6) (width 0.2) (layer "F.Cu") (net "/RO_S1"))
 (segment (start 111.375 65.46) (end 113.05 67.135) (width 0.2) (layer "F.Cu") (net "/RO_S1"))
 (segment (start 111.211522 90.8) (end 124.95 90.8) (width 0.2) (layer "F.Cu") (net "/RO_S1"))
 (segment (start 113.45 62.455) (end 113.45 82.8) (width 0.2) (layer "F.Cu") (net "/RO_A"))
 (segment (start 111.375 60.38) (end 113.45 62.455) (width 0.2) (layer "F.Cu") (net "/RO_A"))
 (segment (start 113.45 82.8) (end 111.75 84.5) (width 0.2) (layer "F.Cu") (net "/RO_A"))
 (segment (start 126.625 75.62) (end 129.829448 75.62) (width 0.2) (layer "F.Cu") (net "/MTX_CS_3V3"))
 (segment (start 129.829448 75.62) (end 136.179448 69.27) (width 0.2) (layer "F.Cu") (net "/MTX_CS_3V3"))
 (segment (start 136.179448 69.27) (end 136.525 69.27) (width 0.2) (layer "F.Cu") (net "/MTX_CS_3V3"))
 (segment (start 133.010001 68) (end 135.550001 65.46) (width 0.2) (layer "F.Cu") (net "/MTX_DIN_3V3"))
 (segment (start 126.625 68) (end 133.010001 68) (width 0.2) (layer "F.Cu") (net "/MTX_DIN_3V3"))
 (segment (start 135.550001 65.46) (end 136.525 65.46) (width 0.2) (layer "F.Cu") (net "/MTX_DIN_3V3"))
 (segment (start 141.015 71) (end 141.475 70.54) (width 0.2) (layer "F.Cu") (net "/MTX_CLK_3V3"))
 (segment (start 140 71) (end 141.015 71) (width 0.2) (layer "F.Cu") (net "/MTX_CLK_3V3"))
 (via (at 140 71) (size 0.6) (drill 0.3) (layers "F.Cu" "B.Cu") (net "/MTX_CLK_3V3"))
 (segment (start 137.92 73.08) (end 140 71) (width 0.2) (layer "B.Cu") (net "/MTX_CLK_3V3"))
 (segment (start 126.625 73.08) (end 137.92 73.08) (width 0.2) (layer "B.Cu") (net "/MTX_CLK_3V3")))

